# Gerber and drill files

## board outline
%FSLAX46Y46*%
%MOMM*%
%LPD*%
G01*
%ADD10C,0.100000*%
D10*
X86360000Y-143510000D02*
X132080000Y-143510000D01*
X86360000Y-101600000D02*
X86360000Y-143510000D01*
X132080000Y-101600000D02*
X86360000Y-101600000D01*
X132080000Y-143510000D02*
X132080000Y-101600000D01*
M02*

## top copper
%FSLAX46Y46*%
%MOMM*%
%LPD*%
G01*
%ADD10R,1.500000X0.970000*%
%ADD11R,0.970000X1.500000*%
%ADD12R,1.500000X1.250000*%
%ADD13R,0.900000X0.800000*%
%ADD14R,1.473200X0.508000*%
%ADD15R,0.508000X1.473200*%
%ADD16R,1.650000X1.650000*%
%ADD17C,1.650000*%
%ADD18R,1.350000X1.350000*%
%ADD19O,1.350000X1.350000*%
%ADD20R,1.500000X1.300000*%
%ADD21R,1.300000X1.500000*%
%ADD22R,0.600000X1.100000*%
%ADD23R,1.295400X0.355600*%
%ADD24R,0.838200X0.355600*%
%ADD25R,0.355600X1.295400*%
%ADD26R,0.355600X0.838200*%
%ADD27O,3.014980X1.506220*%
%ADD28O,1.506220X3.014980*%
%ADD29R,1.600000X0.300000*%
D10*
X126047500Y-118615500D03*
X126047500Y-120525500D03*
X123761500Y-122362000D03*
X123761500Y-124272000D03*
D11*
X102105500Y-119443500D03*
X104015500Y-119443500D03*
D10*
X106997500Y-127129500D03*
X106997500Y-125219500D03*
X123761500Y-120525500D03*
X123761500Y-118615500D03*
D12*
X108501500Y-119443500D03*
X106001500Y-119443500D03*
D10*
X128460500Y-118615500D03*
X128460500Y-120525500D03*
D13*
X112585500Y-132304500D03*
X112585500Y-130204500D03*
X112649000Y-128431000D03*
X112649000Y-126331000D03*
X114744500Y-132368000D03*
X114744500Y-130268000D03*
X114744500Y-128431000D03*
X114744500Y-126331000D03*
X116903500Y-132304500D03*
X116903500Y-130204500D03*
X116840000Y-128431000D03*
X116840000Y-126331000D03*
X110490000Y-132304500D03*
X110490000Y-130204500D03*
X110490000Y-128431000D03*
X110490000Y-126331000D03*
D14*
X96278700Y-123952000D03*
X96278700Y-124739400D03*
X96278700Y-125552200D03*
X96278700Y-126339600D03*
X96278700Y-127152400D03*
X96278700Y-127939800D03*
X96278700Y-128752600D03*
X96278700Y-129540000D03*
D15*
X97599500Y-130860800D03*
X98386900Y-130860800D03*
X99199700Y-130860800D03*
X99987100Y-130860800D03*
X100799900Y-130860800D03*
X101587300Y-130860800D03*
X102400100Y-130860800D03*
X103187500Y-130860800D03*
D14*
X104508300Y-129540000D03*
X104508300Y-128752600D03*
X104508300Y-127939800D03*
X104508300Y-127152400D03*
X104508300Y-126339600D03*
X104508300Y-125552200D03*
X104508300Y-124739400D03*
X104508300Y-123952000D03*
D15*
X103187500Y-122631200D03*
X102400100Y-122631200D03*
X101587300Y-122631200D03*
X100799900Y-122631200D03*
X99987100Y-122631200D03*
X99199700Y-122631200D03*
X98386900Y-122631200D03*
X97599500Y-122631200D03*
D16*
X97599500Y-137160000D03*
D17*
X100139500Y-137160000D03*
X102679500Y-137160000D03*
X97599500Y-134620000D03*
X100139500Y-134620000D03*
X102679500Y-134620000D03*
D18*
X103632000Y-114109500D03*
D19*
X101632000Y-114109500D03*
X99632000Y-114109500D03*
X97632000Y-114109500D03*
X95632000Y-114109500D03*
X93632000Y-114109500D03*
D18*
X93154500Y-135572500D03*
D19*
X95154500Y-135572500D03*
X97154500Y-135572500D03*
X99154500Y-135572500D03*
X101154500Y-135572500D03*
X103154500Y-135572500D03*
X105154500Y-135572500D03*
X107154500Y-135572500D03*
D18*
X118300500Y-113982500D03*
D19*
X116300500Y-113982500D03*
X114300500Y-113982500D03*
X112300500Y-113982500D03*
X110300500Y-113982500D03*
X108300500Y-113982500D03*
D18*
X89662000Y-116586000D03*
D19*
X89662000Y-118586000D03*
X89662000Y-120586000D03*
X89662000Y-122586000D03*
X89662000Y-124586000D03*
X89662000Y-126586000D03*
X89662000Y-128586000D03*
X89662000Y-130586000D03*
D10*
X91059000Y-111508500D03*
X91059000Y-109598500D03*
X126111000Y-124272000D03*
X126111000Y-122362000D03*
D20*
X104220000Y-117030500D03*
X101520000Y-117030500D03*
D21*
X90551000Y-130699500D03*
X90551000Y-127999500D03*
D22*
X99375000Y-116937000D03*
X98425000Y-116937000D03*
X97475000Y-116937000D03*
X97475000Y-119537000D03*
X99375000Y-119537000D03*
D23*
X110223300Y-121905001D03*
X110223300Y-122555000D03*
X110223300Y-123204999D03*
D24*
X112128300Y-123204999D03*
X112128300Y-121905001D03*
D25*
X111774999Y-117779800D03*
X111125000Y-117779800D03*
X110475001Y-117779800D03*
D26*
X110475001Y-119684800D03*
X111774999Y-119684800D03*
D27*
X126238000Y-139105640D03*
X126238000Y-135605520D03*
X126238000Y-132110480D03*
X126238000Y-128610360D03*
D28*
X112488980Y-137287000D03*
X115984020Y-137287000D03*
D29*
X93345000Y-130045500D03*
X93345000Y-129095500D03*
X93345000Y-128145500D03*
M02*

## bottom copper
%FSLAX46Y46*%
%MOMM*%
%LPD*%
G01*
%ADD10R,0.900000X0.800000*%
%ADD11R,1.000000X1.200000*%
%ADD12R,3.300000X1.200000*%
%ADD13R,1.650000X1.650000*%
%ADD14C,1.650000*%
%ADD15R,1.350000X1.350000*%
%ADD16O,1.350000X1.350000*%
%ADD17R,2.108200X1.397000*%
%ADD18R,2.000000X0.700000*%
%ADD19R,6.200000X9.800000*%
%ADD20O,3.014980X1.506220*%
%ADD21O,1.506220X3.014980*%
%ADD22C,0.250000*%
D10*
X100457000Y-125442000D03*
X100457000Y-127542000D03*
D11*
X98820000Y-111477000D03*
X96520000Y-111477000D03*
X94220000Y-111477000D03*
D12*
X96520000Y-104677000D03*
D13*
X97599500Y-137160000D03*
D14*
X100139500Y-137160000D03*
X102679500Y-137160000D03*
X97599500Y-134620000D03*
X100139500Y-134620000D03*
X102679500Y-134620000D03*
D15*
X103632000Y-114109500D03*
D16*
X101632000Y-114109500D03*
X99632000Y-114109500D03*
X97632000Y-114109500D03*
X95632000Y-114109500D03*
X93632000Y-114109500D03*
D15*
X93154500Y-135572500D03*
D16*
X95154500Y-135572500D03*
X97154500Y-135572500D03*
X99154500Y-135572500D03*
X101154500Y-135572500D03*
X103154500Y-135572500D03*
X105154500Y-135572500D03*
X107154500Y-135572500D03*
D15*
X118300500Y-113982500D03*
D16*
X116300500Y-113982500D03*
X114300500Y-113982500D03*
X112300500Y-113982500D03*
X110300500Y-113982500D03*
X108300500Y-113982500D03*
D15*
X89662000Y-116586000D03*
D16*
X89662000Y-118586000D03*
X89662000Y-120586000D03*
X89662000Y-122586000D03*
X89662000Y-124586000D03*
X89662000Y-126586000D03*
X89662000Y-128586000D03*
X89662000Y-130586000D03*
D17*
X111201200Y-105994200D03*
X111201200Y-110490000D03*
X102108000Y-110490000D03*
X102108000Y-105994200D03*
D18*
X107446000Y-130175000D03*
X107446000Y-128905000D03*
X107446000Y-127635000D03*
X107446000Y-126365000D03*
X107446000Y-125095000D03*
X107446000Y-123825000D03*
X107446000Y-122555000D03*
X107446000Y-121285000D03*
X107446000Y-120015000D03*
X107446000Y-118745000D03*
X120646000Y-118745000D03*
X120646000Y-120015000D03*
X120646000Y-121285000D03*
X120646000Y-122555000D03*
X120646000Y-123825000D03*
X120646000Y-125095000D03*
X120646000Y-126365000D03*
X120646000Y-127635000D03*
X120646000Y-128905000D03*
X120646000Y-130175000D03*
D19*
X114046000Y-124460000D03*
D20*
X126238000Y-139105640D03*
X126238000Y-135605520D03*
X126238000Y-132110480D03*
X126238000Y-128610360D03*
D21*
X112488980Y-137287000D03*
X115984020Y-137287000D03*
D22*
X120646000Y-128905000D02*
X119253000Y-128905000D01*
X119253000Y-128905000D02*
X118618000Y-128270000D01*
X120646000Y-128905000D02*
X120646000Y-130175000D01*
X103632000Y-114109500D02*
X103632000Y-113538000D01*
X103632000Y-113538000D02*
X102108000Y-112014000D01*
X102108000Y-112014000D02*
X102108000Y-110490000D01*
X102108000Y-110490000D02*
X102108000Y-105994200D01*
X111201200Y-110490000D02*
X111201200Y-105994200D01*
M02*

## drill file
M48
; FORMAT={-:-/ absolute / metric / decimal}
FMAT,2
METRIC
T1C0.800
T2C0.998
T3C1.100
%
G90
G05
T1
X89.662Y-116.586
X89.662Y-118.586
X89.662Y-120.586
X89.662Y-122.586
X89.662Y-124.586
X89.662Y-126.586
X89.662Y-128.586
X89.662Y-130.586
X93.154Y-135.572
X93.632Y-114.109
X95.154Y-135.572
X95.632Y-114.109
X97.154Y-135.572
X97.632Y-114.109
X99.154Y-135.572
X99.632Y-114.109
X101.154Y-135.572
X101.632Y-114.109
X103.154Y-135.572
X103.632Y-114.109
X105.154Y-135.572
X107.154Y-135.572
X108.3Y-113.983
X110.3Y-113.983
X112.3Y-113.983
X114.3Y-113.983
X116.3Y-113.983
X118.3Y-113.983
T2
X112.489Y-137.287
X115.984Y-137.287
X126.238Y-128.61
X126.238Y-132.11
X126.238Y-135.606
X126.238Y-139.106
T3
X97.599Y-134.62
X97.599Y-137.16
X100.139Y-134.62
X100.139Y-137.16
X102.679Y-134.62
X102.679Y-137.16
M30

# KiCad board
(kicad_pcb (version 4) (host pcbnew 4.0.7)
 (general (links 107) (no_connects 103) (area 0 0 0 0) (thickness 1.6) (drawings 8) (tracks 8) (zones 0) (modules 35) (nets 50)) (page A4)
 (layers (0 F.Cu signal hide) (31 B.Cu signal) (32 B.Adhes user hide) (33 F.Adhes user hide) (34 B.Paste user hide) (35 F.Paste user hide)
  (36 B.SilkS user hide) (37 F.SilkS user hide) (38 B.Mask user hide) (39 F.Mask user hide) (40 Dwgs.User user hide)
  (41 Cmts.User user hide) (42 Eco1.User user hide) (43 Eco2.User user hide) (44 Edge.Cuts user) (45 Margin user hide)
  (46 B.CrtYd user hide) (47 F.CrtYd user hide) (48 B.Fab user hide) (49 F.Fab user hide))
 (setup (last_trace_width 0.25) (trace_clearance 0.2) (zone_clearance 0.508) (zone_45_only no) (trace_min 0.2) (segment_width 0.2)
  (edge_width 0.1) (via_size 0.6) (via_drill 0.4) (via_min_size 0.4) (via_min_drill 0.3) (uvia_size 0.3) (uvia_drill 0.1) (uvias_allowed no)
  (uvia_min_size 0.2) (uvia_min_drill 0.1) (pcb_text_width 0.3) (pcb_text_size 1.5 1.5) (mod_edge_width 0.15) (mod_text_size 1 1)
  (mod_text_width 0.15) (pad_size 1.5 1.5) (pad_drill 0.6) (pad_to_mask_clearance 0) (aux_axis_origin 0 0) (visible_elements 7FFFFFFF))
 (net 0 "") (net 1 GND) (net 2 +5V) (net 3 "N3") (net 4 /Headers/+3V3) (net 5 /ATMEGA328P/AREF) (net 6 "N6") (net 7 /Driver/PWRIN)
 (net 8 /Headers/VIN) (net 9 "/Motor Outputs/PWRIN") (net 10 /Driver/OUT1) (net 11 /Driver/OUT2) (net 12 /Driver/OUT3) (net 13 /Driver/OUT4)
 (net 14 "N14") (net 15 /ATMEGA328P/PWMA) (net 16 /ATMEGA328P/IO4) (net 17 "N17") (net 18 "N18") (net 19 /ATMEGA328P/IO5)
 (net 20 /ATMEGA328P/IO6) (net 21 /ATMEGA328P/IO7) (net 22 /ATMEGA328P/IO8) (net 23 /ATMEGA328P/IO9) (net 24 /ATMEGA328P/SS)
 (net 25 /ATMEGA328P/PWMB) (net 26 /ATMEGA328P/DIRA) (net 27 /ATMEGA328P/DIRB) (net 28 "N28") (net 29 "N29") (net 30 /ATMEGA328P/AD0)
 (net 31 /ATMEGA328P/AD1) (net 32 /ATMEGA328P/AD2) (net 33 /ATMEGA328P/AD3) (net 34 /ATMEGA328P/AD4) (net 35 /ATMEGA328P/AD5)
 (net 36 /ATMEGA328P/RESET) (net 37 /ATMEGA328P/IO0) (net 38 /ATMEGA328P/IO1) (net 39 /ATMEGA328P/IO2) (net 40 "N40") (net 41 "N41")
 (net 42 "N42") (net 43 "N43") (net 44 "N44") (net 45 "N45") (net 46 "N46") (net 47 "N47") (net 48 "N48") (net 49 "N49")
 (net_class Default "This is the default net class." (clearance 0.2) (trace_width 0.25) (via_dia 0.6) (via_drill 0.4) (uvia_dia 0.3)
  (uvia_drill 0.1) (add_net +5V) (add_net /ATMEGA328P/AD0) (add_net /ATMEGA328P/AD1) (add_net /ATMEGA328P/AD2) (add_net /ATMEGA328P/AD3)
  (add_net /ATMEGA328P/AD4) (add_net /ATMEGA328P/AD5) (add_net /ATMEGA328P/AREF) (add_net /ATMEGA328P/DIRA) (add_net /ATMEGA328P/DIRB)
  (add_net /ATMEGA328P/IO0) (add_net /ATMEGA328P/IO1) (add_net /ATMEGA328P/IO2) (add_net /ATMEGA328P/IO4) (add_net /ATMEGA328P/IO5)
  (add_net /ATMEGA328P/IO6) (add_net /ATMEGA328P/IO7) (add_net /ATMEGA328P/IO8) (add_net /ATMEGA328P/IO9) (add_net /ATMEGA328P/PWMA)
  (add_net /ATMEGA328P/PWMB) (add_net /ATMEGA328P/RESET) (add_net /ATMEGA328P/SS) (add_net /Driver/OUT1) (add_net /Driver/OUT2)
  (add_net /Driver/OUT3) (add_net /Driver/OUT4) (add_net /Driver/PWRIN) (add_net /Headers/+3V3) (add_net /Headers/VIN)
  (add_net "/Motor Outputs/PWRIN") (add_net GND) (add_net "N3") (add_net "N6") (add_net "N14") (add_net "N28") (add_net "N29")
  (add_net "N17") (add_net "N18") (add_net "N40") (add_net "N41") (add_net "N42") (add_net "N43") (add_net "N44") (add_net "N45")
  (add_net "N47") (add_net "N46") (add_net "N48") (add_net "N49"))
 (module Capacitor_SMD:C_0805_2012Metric (layer F.Cu) (at 126.0475 119.5705 270)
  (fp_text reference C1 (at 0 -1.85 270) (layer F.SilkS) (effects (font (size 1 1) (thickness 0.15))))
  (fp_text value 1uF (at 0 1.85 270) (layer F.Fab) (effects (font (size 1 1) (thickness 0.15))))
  (pad 1 smd rect (at -0.955 0 270) (size 0.97 1.5) (layers F.Cu F.Paste F.Mask) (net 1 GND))
  (pad 2 smd rect (at 0.955 0 270) (size 0.97 1.5) (layers F.Cu F.Paste F.Mask) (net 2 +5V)))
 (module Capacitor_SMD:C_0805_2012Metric (layer F.Cu) (at 123.7615 123.317 270)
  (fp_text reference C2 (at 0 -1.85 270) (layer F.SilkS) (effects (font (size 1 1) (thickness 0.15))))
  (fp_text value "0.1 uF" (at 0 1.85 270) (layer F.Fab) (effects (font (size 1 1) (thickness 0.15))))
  (pad 1 smd rect (at -0.955 0 270) (size 0.97 1.5) (layers F.Cu F.Paste F.Mask) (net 2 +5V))
  (pad 2 smd rect (at 0.955 0 270) (size 0.97 1.5) (layers F.Cu F.Paste F.Mask) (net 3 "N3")))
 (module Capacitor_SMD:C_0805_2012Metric (layer F.Cu) (at 103.0605 119.4435)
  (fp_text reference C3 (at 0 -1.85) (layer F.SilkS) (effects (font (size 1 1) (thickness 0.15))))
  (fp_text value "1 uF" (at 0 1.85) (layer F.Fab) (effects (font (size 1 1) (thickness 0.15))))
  (pad 1 smd rect (at -0.955 0) (size 0.97 1.5) (layers F.Cu F.Paste F.Mask) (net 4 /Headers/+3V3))
  (pad 2 smd rect (at 0.955 0) (size 0.97 1.5) (layers F.Cu F.Paste F.Mask) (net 1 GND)))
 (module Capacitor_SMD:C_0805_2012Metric (layer F.Cu) (at 106.9975 126.1745 90)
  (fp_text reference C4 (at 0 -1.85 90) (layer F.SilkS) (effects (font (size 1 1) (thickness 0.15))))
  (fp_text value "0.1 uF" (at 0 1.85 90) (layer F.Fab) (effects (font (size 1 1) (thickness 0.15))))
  (pad 1 smd rect (at -0.955 0 90) (size 0.97 1.5) (layers F.Cu F.Paste F.Mask) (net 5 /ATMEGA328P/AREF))
  (pad 2 smd rect (at 0.955 0 90) (size 0.97 1.5) (layers F.Cu F.Paste F.Mask) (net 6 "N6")))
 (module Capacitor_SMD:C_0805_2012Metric (layer F.Cu) (at 123.7615 119.5705 90)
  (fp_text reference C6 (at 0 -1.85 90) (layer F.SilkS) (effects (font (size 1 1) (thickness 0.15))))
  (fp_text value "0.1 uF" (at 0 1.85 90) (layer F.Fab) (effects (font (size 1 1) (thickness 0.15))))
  (pad 1 smd rect (at -0.955 0 90) (size 0.97 1.5) (layers F.Cu F.Paste F.Mask) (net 2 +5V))
  (pad 2 smd rect (at 0.955 0 90) (size 0.97 1.5) (layers F.Cu F.Paste F.Mask) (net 1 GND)))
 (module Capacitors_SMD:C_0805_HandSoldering (layer F.Cu) (at 107.2515 119.4435 180)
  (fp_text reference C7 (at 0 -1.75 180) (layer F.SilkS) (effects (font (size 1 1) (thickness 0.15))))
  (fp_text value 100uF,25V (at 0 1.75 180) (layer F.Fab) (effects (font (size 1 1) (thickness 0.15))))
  (pad 1 smd rect (at -1.25 0 180) (size 1.5 1.25) (layers F.Cu F.Paste F.Mask) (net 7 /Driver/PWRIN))
  (pad 2 smd rect (at 1.25 0 180) (size 1.5 1.25) (layers F.Cu F.Paste F.Mask) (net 1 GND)))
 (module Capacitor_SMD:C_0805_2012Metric (layer F.Cu) (at 128.4605 119.5705 270)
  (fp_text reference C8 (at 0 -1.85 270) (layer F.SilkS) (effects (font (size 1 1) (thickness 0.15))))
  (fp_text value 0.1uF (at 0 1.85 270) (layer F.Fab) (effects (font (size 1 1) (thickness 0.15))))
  (pad 1 smd rect (at -0.955 0 270) (size 0.97 1.5) (layers F.Cu F.Paste F.Mask) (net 1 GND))
  (pad 2 smd rect (at 0.955 0 270) (size 0.97 1.5) (layers F.Cu F.Paste F.Mask) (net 2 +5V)))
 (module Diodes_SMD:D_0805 (layer B.Cu) (at 100.457 126.492 270)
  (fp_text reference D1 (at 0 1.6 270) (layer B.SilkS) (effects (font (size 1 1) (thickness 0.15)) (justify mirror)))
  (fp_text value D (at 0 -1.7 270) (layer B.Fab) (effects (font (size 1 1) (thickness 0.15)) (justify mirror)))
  (pad 1 smd rect (at -1.05 0 270) (size 0.8 0.9) (layers B.Cu B.Paste B.Mask) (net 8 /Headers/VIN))
  (pad 2 smd rect (at 1.05 0 270) (size 0.8 0.9) (layers B.Cu B.Paste B.Mask) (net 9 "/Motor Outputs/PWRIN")))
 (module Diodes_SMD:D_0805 (layer F.Cu) (at 112.5855 131.2545 90)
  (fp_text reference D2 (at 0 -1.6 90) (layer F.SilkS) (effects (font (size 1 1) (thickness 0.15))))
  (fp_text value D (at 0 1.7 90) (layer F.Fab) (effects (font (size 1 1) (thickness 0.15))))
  (pad 1 smd rect (at -1.05 0 90) (size 0.8 0.9) (layers F.Cu F.Paste F.Mask) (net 9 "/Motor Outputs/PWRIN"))
  (pad 2 smd rect (at 1.05 0 90) (size 0.8 0.9) (layers F.Cu F.Paste F.Mask) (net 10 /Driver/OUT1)))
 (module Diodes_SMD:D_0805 (layer F.Cu) (at 112.649 127.381 90)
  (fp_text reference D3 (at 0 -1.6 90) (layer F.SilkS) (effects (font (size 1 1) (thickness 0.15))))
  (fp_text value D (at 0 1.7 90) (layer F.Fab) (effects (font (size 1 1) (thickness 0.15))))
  (pad 1 smd rect (at -1.05 0 90) (size 0.8 0.9) (layers F.Cu F.Paste F.Mask) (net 10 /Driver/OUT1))
  (pad 2 smd rect (at 1.05 0 90) (size 0.8 0.9) (layers F.Cu F.Paste F.Mask) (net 1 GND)))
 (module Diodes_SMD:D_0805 (layer F.Cu) (at 114.7445 131.318 90)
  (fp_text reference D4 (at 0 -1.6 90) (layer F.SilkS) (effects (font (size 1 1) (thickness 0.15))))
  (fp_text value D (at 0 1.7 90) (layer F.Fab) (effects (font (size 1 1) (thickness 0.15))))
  (pad 1 smd rect (at -1.05 0 90) (size 0.8 0.9) (layers F.Cu F.Paste F.Mask) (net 9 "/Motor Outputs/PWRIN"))
  (pad 2 smd rect (at 1.05 0 90) (size 0.8 0.9) (layers F.Cu F.Paste F.Mask) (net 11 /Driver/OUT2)))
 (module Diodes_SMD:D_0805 (layer F.Cu) (at 114.7445 127.381 90)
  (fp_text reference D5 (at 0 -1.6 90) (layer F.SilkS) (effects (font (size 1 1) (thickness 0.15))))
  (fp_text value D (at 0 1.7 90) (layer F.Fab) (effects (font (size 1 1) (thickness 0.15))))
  (pad 1 smd rect (at -1.05 0 90) (size 0.8 0.9) (layers F.Cu F.Paste F.Mask) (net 11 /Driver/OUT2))
  (pad 2 smd rect (at 1.05 0 90) (size 0.8 0.9) (layers F.Cu F.Paste F.Mask) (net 1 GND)))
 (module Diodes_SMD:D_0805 (layer F.Cu) (at 116.9035 131.2545 90)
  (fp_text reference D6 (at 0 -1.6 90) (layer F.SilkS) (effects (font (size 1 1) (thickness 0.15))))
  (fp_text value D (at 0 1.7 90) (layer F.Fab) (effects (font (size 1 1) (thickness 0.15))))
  (pad 1 smd rect (at -1.05 0 90) (size 0.8 0.9) (layers F.Cu F.Paste F.Mask) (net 9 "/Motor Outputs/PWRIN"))
  (pad 2 smd rect (at 1.05 0 90) (size 0.8 0.9) (layers F.Cu F.Paste F.Mask) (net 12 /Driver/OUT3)))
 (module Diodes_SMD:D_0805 (layer F.Cu) (at 116.84 127.381 90)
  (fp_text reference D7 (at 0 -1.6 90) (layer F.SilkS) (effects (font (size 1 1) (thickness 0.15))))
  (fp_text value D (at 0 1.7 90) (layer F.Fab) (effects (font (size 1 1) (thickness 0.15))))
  (pad 1 smd rect (at -1.05 0 90) (size 0.8 0.9) (layers F.Cu F.Paste F.Mask) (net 12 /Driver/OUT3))
  (pad 2 smd rect (at 1.05 0 90) (size 0.8 0.9) (layers F.Cu F.Paste F.Mask) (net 1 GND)))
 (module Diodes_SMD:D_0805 (layer F.Cu) (at 110.49 131.2545 90)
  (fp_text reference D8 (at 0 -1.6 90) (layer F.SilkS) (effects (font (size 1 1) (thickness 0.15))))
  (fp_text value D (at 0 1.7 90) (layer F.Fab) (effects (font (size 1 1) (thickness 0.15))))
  (pad 1 smd rect (at -1.05 0 90) (size 0.8 0.9) (layers F.Cu F.Paste F.Mask) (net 9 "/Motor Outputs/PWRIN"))
  (pad 2 smd rect (at 1.05 0 90) (size 0.8 0.9) (layers F.Cu F.Paste F.Mask) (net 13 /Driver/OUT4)))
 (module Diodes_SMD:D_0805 (layer F.Cu) (at 110.49 127.381 90)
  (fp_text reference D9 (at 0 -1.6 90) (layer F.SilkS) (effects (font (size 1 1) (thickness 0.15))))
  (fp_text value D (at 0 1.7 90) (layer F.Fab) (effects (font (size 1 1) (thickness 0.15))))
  (pad 1 smd rect (at -1.05 0 90) (size 0.8 0.9) (layers F.Cu F.Paste F.Mask) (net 13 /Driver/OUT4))
  (pad 2 smd rect (at 1.05 0 90) (size 0.8 0.9) (layers F.Cu F.Paste F.Mask) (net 1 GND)))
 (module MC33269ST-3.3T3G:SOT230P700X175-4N (layer B.Cu) (at 96.52 108.077 90)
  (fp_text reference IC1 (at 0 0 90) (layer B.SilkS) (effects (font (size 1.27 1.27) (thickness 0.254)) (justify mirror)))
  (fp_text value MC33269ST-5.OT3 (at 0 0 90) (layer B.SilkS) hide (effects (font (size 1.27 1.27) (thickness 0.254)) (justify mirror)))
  (pad 1 smd rect (at -3.4 2.3) (size 1 1.2) (layers B.Cu B.Paste B.Mask) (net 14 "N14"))
  (pad 2 smd rect (at -3.4 0) (size 1 1.2) (layers B.Cu B.Paste B.Mask) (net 2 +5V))
  (pad 3 smd rect (at -3.4 -2.3) (size 1 1.2) (layers B.Cu B.Paste B.Mask) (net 8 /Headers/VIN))
  (pad 4 smd rect (at 3.4 0 90) (size 1.2 3.3) (layers B.Cu B.Paste B.Mask) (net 2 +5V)))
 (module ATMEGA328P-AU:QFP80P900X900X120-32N (layer F.Cu) (at 100.3935 126.746)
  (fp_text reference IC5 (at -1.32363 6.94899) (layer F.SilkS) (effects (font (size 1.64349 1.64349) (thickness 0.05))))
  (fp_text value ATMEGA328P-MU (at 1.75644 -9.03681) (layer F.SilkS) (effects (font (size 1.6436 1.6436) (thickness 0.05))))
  (pad 1 smd rect (at -4.1148 -2.794 270) (size 0.508 1.4732) (layers F.Cu F.Paste F.Mask) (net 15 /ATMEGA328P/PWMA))
  (pad 2 smd rect (at -4.1148 -2.0066 270) (size 0.508 1.4732) (layers F.Cu F.Paste F.Mask) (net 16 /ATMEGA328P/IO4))
  (pad 3 smd rect (at -4.1148 -1.1938 270) (size 0.508 1.4732) (layers F.Cu F.Paste F.Mask) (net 1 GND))
  (pad 4 smd rect (at -4.1148 -0.4064 270) (size 0.508 1.4732) (layers F.Cu F.Paste F.Mask) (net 2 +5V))
  (pad 5 smd rect (at -4.1148 0.4064 270) (size 0.508 1.4732) (layers F.Cu F.Paste F.Mask) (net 1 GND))
  (pad 6 smd rect (at -4.1148 1.1938 270) (size 0.508 1.4732) (layers F.Cu F.Paste F.Mask) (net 2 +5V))
  (pad 7 smd rect (at -4.1148 2.0066 270) (size 0.508 1.4732) (layers F.Cu F.Paste F.Mask) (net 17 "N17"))
  (pad 8 smd rect (at -4.1148 2.794 270) (size 0.508 1.4732) (layers F.Cu F.Paste F.Mask) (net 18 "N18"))
  (pad 9 smd rect (at -2.794 4.1148 180) (size 0.508 1.4732) (layers F.Cu F.Paste F.Mask) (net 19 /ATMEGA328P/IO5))
  (pad 10 smd rect (at -2.0066 4.1148 180) (size 0.508 1.4732) (layers F.Cu F.Paste F.Mask) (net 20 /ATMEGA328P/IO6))
  (pad 11 smd rect (at -1.1938 4.1148 180) (size 0.508 1.4732) (layers F.Cu F.Paste F.Mask) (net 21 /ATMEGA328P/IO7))
  (pad 12 smd rect (at -0.4064 4.1148 180) (size 0.508 1.4732) (layers F.Cu F.Paste F.Mask) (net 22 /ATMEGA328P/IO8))
  (pad 13 smd rect (at 0.4064 4.1148 180) (size 0.508 1.4732) (layers F.Cu F.Paste F.Mask) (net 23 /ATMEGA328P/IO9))
  (pad 14 smd rect (at 1.1938 4.1148 180) (size 0.508 1.4732) (layers F.Cu F.Paste F.Mask) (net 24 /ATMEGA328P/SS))
  (pad 15 smd rect (at 2.0066 4.1148 180) (size 0.508 1.4732) (layers F.Cu F.Paste F.Mask) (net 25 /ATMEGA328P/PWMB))
  (pad 16 smd rect (at 2.794 4.1148 180) (size 0.508 1.4732) (layers F.Cu F.Paste F.Mask) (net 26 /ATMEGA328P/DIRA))
  (pad 17 smd rect (at 4.1148 2.794 270) (size 0.508 1.4732) (layers F.Cu F.Paste F.Mask) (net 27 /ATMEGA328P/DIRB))
  (pad 18 smd rect (at 4.1148 2.0066 270) (size 0.508 1.4732) (layers F.Cu F.Paste F.Mask) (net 2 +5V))
  (pad 19 smd rect (at 4.1148 1.1938 270) (size 0.508 1.4732) (layers F.Cu F.Paste F.Mask) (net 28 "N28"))
  (pad 20 smd rect (at 4.1148 0.4064 270) (size 0.508 1.4732) (layers F.Cu F.Paste F.Mask) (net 5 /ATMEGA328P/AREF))
  (pad 21 smd rect (at 4.1148 -0.4064 270) (size 0.508 1.4732) (layers F.Cu F.Paste F.Mask) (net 1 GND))
  (pad 22 smd rect (at 4.1148 -1.1938 270) (size 0.508 1.4732) (layers F.Cu F.Paste F.Mask) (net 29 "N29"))
  (pad 23 smd rect (at 4.1148 -2.0066 270) (size 0.508 1.4732) (layers F.Cu F.Paste F.Mask) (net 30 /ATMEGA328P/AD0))
  (pad 24 smd rect (at 4.1148 -2.794 270) (size 0.508 1.4732) (layers F.Cu F.Paste F.Mask) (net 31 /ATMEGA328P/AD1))
  (pad 25 smd rect (at 2.794 -4.1148 180) (size 0.508 1.4732) (layers F.Cu F.Paste F.Mask) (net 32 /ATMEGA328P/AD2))
  (pad 26 smd rect (at 2.0066 -4.1148 180) (size 0.508 1.4732) (layers F.Cu F.Paste F.Mask) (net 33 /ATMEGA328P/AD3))
  (pad 27 smd rect (at 1.1938 -4.1148 180) (size 0.508 1.4732) (layers F.Cu F.Paste F.Mask) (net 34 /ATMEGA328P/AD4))
  (pad 28 smd rect (at 0.4064 -4.1148 180) (size 0.508 1.4732) (layers F.Cu F.Paste F.Mask) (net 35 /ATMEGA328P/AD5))
  (pad 29 smd rect (at -0.4064 -4.1148 180) (size 0.508 1.4732) (layers F.Cu F.Paste F.Mask) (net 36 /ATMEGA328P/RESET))
  (pad 30 smd rect (at -1.1938 -4.1148 180) (size 0.508 1.4732) (layers F.Cu F.Paste F.Mask) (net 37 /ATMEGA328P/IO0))
  (pad 31 smd rect (at -2.0066 -4.1148 180) (size 0.508 1.4732) (layers F.Cu F.Paste F.Mask) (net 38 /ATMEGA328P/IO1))
  (pad 32 smd rect (at -2.794 -4.1148 180) (size 0.508 1.4732) (layers F.Cu F.Paste F.Mask) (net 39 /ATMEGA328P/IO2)))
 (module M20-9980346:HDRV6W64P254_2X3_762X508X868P (layer F.Cu) (at 97.5995 137.16)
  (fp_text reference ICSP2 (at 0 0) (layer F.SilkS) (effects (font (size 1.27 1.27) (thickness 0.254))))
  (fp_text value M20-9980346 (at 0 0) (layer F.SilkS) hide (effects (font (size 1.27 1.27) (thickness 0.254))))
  (pad 1 thru_hole rect (at 0 0 90) (size 1.65 1.65) (drill 1.1) (layers *.Cu *.Mask F.SilkS) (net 26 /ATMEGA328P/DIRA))
  (pad 3 thru_hole circle (at 2.54 0 90) (size 1.65 1.65) (drill 1.1) (layers *.Cu *.Mask F.SilkS) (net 27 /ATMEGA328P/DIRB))
  (pad 5 thru_hole circle (at 5.08 0 90) (size 1.65 1.65) (drill 1.1) (layers *.Cu *.Mask F.SilkS) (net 36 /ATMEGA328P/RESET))
  (pad 2 thru_hole circle (at 0 -2.54 90) (size 1.65 1.65) (drill 1.1) (layers *.Cu *.Mask F.SilkS) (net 2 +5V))
  (pad 4 thru_hole circle (at 2.54 -2.54 90) (size 1.65 1.65) (drill 1.1) (layers *.Cu *.Mask F.SilkS) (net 25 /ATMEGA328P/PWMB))
  (pad 6 thru_hole circle (at 5.08 -2.54 90) (size 1.65 1.65) (drill 1.1) (layers *.Cu *.Mask F.SilkS) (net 1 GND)))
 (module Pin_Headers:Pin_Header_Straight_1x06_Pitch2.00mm (layer B.Cu) (at 103.632 114.1095 90)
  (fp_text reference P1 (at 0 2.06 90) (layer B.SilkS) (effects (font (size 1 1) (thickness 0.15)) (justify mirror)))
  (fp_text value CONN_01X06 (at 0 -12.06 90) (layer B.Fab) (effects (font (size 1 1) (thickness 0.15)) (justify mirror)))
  (pad 1 thru_hole rect (at 0 0 90) (size 1.35 1.35) (drill 0.8) (layers *.Cu *.Mask) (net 36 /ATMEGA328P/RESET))
  (pad 2 thru_hole oval (at 0 -2 90) (size 1.35 1.35) (drill 0.8) (layers *.Cu *.Mask) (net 4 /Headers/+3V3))
  (pad 3 thru_hole oval (at 0 -4 90) (size 1.35 1.35) (drill 0.8) (layers *.Cu *.Mask) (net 2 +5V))
  (pad 4 thru_hole oval (at 0 -6 90) (size 1.35 1.35) (drill 0.8) (layers *.Cu *.Mask) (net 1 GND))
  (pad 5 thru_hole oval (at 0 -8 90) (size 1.35 1.35) (drill 0.8) (layers *.Cu *.Mask) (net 1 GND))
  (pad 6 thru_hole oval (at 0 -10 90) (size 1.35 1.35) (drill 0.8) (layers *.Cu *.Mask) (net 8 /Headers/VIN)))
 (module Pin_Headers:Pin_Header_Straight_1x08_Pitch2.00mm (layer B.Cu) (at 93.1545 135.5725 270)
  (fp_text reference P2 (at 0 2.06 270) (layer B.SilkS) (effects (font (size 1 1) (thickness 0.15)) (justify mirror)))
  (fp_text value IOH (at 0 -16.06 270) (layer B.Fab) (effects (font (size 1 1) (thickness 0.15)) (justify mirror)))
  (pad 1 thru_hole rect (at 0 0 270) (size 1.35 1.35) (drill 0.8) (layers *.Cu *.Mask) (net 22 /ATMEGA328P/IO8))
  (pad 2 thru_hole oval (at 0 -2 270) (size 1.35 1.35) (drill 0.8) (layers *.Cu *.Mask) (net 23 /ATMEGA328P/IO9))
  (pad 3 thru_hole oval (at 0 -4 270) (size 1.35 1.35) (drill 0.8) (layers *.Cu *.Mask) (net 24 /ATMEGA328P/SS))
  (pad 4 thru_hole oval (at 0 -6 270) (size 1.35 1.35) (drill 0.8) (layers *.Cu *.Mask) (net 25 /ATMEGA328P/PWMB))
  (pad 5 thru_hole oval (at 0 -8 270) (size 1.35 1.35) (drill 0.8) (layers *.Cu *.Mask) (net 26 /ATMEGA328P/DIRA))
  (pad 6 thru_hole oval (at 0 -10 270) (size 1.35 1.35) (drill 0.8) (layers *.Cu *.Mask) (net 27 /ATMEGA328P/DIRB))
  (pad 7 thru_hole oval (at 0 -12 270) (size 1.35 1.35) (drill 0.8) (layers *.Cu *.Mask) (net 1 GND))
  (pad 8 thru_hole oval (at 0 -14 270) (size 1.35 1.35) (drill 0.8) (layers *.Cu *.Mask) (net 5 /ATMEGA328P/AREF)))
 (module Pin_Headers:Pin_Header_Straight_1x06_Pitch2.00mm (layer F.Cu) (at 118.3005 113.9825 270)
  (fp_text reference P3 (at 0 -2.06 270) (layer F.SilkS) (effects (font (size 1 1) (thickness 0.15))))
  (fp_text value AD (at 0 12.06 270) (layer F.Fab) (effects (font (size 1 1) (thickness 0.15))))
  (pad 1 thru_hole rect (at 0 0 270) (size 1.35 1.35) (drill 0.8) (layers *.Cu *.Mask) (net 30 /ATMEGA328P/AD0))
  (pad 2 thru_hole oval (at 0 2 270) (size 1.35 1.35) (drill 0.8) (layers *.Cu *.Mask) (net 31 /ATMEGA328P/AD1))
  (pad 3 thru_hole oval (at 0 4 270) (size 1.35 1.35) (drill 0.8) (layers *.Cu *.Mask) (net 32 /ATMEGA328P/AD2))
  (pad 4 thru_hole oval (at 0 6 270) (size 1.35 1.35) (drill 0.8) (layers *.Cu *.Mask) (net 33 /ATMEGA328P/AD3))
  (pad 5 thru_hole oval (at 0 8 270) (size 1.35 1.35) (drill 0.8) (layers *.Cu *.Mask) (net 34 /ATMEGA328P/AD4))
  (pad 6 thru_hole oval (at 0 10 270) (size 1.35 1.35) (drill 0.8) (layers *.Cu *.Mask) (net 35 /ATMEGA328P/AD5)))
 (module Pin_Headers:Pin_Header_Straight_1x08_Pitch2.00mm (layer B.Cu) (at 89.662 116.586 180)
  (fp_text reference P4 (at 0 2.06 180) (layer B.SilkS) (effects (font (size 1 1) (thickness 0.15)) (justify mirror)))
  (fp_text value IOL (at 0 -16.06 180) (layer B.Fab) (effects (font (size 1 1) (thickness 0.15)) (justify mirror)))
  (pad 1 thru_hole rect (at 0 0 180) (size 1.35 1.35) (drill 0.8) (layers *.Cu *.Mask) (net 37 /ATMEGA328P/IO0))
  (pad 2 thru_hole oval (at 0 -2 180) (size 1.35 1.35) (drill 0.8) (layers *.Cu *.Mask) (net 38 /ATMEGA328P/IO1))
  (pad 3 thru_hole oval (at 0 -4 180) (size 1.35 1.35) (drill 0.8) (layers *.Cu *.Mask) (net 39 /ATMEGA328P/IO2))
  (pad 4 thru_hole oval (at 0 -6 180) (size 1.35 1.35) (drill 0.8) (layers *.Cu *.Mask) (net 15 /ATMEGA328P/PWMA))
  (pad 5 thru_hole oval (at 0 -8 180) (size 1.35 1.35) (drill 0.8) (layers *.Cu *.Mask) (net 16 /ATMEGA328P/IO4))
  (pad 6 thru_hole oval (at 0 -10 180) (size 1.35 1.35) (drill 0.8) (layers *.Cu *.Mask) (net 19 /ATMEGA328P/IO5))
  (pad 7 thru_hole oval (at 0 -12 180) (size 1.35 1.35) (drill 0.8) (layers *.Cu *.Mask) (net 20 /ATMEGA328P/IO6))
  (pad 8 thru_hole oval (at 0 -14 180) (size 1.35 1.35) (drill 0.8) (layers *.Cu *.Mask) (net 21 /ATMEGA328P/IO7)))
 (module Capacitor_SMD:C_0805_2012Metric (layer F.Cu) (at 91.059 110.5535 90)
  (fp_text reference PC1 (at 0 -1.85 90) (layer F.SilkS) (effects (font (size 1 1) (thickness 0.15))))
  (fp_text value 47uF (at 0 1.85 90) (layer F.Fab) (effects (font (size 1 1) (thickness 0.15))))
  (pad 1 smd rect (at -0.955 0 90) (size 0.97 1.5) (layers F.Cu F.Paste F.Mask) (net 8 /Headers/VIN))
  (pad 2 smd rect (at 0.955 0 90) (size 0.97 1.5) (layers F.Cu F.Paste F.Mask) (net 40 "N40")))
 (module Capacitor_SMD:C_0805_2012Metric (layer F.Cu) (at 126.111 123.317 90)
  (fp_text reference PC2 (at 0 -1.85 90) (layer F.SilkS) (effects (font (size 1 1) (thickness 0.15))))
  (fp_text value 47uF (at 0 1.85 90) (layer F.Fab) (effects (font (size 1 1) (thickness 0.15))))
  (pad 1 smd rect (at -0.955 0 90) (size 0.97 1.5) (layers F.Cu F.Paste F.Mask) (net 2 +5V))
  (pad 2 smd rect (at 0.955 0 90) (size 0.97 1.5) (layers F.Cu F.Paste F.Mask) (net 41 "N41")))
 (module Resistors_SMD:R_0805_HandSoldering (layer F.Cu) (at 102.87 117.0305 180)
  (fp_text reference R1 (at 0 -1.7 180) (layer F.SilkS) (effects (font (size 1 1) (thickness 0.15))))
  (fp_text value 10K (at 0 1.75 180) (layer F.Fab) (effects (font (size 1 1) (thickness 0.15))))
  (pad 1 smd rect (at -1.35 0 180) (size 1.5 1.3) (layers F.Cu F.Paste F.Mask) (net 36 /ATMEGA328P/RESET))
  (pad 2 smd rect (at 1.35 0 180) (size 1.5 1.3) (layers F.Cu F.Paste F.Mask) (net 2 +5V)))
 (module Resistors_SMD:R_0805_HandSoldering (layer F.Cu) (at 90.551 129.3495 90)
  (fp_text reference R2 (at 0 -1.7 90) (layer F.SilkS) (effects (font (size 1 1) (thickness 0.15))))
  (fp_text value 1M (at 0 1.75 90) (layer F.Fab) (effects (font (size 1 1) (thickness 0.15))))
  (pad 1 smd rect (at -1.35 0 90) (size 1.5 1.3) (layers F.Cu F.Paste F.Mask) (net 18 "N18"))
  (pad 2 smd rect (at 1.35 0 90) (size 1.5 1.3) (layers F.Cu F.Paste F.Mask) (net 17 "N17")))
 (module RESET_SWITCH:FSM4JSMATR (layer B.Cu) (at 102.108 110.49 180)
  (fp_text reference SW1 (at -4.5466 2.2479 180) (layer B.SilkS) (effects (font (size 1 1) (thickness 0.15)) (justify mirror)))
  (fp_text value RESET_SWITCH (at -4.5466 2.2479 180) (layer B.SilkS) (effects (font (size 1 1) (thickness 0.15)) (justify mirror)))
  (pad 1 smd rect (at -9.0932 4.4958 180) (size 2.1082 1.397) (layers B.Cu B.Paste B.Mask) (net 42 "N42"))
  (pad 2 smd rect (at -9.0932 0 180) (size 2.1082 1.397) (layers B.Cu B.Paste B.Mask) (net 42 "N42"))
  (pad 3 smd rect (at 0 0 180) (size 2.1082 1.397) (layers B.Cu B.Paste B.Mask) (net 36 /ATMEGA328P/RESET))
  (pad 4 smd rect (at 0 4.4958 180) (size 2.1082 1.397) (layers B.Cu B.Paste B.Mask) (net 36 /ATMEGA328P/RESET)))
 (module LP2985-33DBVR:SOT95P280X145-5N (layer F.Cu) (at 98.425 118.237 270)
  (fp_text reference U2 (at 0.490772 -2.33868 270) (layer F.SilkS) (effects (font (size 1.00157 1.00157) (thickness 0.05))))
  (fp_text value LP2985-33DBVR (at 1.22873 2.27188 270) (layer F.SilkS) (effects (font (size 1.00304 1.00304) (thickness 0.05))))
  (pad 1 smd rect (at -1.3 -0.95 270) (size 1.1 0.6) (layers F.Cu F.Paste F.Mask) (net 2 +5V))
  (pad 2 smd rect (at -1.3 0 270) (size 1.1 0.6) (layers F.Cu F.Paste F.Mask) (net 1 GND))
  (pad 3 smd rect (at -1.3 0.95 270) (size 1.1 0.6) (layers F.Cu F.Paste F.Mask) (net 2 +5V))
  (pad 4 smd rect (at 1.3 0.95 90) (size 1.1 0.6) (layers F.Cu F.Paste F.Mask) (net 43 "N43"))
  (pad 5 smd rect (at 1.3 -0.95 90) (size 1.1 0.6) (layers F.Cu F.Paste F.Mask) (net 4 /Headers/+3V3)))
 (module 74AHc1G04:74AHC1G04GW (layer F.Cu) (at 111.0615 122.555)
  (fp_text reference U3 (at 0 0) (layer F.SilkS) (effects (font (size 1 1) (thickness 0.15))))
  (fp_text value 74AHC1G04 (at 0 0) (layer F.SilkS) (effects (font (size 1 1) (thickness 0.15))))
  (pad 1 smd rect (at -0.8382 -0.649999) (size 1.2954 0.3556) (layers F.Cu F.Paste F.Mask))
  (pad 2 smd rect (at -0.8382 0) (size 1.2954 0.3556) (layers F.Cu F.Paste F.Mask) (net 26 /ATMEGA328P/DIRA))
  (pad 3 smd rect (at -0.8382 0.649999) (size 1.2954 0.3556) (layers F.Cu F.Paste F.Mask) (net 1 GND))
  (pad 4 smd rect (at 1.0668 0.649999) (size 0.8382 0.3556) (layers F.Cu F.Paste F.Mask) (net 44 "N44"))
  (pad 5 smd rect (at 1.0668 -0.649999) (size 0.8382 0.3556) (layers F.Cu F.Paste F.Mask) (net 2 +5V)))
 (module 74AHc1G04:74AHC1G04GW (layer F.Cu) (at 111.125 118.618 270)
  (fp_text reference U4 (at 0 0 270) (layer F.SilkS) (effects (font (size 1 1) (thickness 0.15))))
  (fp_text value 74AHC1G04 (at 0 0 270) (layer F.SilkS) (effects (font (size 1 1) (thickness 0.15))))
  (pad 1 smd rect (at -0.8382 -0.649999 270) (size 1.2954 0.3556) (layers F.Cu F.Paste F.Mask))
  (pad 2 smd rect (at -0.8382 0 270) (size 1.2954 0.3556) (layers F.Cu F.Paste F.Mask) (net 27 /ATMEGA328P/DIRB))
  (pad 3 smd rect (at -0.8382 0.649999 270) (size 1.2954 0.3556) (layers F.Cu F.Paste F.Mask) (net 1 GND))
  (pad 4 smd rect (at 1.0668 0.649999 270) (size 0.8382 0.3556) (layers F.Cu F.Paste F.Mask) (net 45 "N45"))
  (pad 5 smd rect (at 1.0668 -0.649999 270) (size 0.8382 0.3556) (layers F.Cu F.Paste F.Mask) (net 2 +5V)))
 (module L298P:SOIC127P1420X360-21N (layer B.Cu) (at 114.046 124.46)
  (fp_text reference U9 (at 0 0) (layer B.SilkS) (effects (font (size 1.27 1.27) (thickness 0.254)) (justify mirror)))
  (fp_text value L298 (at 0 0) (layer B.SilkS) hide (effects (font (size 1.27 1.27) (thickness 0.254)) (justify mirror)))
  (pad 1 smd rect (at -6.6 5.715 270) (size 0.7 2) (layers B.Cu B.Paste B.Mask) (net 1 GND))
  (pad 2 smd rect (at -6.6 4.445 270) (size 0.7 2) (layers B.Cu B.Paste B.Mask) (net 1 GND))
  (pad 3 smd rect (at -6.6 3.175 270) (size 0.7 2) (layers B.Cu B.Paste B.Mask) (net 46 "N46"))
  (pad 4 smd rect (at -6.6 1.905 270) (size 0.7 2) (layers B.Cu B.Paste B.Mask) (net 10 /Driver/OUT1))
  (pad 5 smd rect (at -6.6 0.635 270) (size 0.7 2) (layers B.Cu B.Paste B.Mask) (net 11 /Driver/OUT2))
  (pad 6 smd rect (at -6.6 -0.635 270) (size 0.7 2) (layers B.Cu B.Paste B.Mask) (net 7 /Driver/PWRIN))
  (pad 7 smd rect (at -6.6 -1.905 270) (size 0.7 2) (layers B.Cu B.Paste B.Mask) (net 26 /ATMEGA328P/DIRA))
  (pad 8 smd rect (at -6.6 -3.175 270) (size 0.7 2) (layers B.Cu B.Paste B.Mask) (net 15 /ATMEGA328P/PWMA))
  (pad 9 smd rect (at -6.6 -4.445 270) (size 0.7 2) (layers B.Cu B.Paste B.Mask) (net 44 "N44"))
  (pad 10 smd rect (at -6.6 -5.715 270) (size 0.7 2) (layers B.Cu B.Paste B.Mask) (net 1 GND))
  (pad 11 smd rect (at 6.6 -5.715 270) (size 0.7 2) (layers B.Cu B.Paste B.Mask) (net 1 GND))
  (pad 12 smd rect (at 6.6 -4.445 270) (size 0.7 2) (layers B.Cu B.Paste B.Mask) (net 2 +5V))
  (pad 13 smd rect (at 6.6 -3.175 270) (size 0.7 2) (layers B.Cu B.Paste B.Mask) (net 27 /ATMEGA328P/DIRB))
  (pad 14 smd rect (at 6.6 -1.905 270) (size 0.7 2) (layers B.Cu B.Paste B.Mask) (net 25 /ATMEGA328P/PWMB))
  (pad 15 smd rect (at 6.6 -0.635 270) (size 0.7 2) (layers B.Cu B.Paste B.Mask) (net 45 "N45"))
  (pad 16 smd rect (at 6.6 0.635 270) (size 0.7 2) (layers B.Cu B.Paste B.Mask) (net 12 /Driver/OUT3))
  (pad 17 smd rect (at 6.6 1.905 270) (size 0.7 2) (layers B.Cu B.Paste B.Mask) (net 13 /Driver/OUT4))
  (pad 18 smd rect (at 6.6 3.175 270) (size 0.7 2) (layers B.Cu B.Paste B.Mask) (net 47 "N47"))
  (pad 19 smd rect (at 6.6 4.445 270) (size 0.7 2) (layers B.Cu B.Paste B.Mask) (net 1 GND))
  (pad 20 smd rect (at 6.6 5.715 270) (size 0.7 2) (layers B.Cu B.Paste B.Mask) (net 1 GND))
  (pad 21 smd rect (at 0 0) (size 6.2 9.8) (layers B.Cu B.Paste B.Mask)))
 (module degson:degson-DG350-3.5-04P (layer B.Cu) (at 126.238 133.858 90)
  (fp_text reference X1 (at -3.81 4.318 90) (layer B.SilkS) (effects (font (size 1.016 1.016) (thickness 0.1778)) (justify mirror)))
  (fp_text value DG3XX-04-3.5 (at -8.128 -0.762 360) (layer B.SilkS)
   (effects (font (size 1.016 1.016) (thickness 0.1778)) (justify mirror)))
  (pad 1 thru_hole oval (at -5.24764 0 270) (size 1.50622 3.01498) (drill 0.99822) (layers *.Cu *.Paste *.Mask) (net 10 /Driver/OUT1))
  (pad 2 thru_hole oval (at -1.74752 0 270) (size 1.50622 3.01498) (drill 0.99822) (layers *.Cu *.Paste *.Mask) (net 11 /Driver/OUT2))
  (pad 3 thru_hole oval (at 1.74752 0 270) (size 1.50622 3.01498) (drill 0.99822) (layers *.Cu *.Paste *.Mask) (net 12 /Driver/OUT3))
  (pad 4 thru_hole oval (at 5.24764 0 270) (size 1.50622 3.01498) (drill 0.99822) (layers *.Cu *.Paste *.Mask) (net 13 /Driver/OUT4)))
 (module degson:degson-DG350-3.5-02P (layer B.Cu) (at 114.2365 137.287)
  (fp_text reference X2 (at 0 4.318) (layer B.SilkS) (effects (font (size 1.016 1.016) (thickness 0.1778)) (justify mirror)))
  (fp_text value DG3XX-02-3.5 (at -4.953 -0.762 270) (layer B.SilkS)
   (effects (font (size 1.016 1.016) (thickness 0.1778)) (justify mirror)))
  (pad 1 thru_hole oval (at -1.74752 0 180) (size 1.50622 3.01498) (drill 0.99822) (layers *.Cu *.Paste *.Mask)
   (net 9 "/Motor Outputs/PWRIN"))
  (pad 2 thru_hole oval (at 1.74752 0 180) (size 1.50622 3.01498) (drill 0.99822) (layers *.Cu *.Paste *.Mask) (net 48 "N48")))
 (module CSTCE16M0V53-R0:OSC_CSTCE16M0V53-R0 (layer F.Cu) (at 93.345 129.0955 90)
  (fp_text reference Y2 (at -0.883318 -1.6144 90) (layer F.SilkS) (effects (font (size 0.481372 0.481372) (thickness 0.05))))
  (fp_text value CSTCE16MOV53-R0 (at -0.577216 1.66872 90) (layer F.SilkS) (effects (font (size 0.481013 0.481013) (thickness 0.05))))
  (pad 1 smd rect (at -0.95 0 180) (size 1.6 0.3) (layers F.Cu F.Paste F.Mask) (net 18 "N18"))
  (pad 2 smd rect (at 0 0 180) (size 1.6 0.3) (layers F.Cu F.Paste F.Mask) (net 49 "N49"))
  (pad 3 smd rect (at 0.95 0 180) (size 1.6 0.3) (layers F.Cu F.Paste F.Mask) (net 17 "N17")))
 (gr_line (start 86.36 143.51) (end 132.08 143.51) (angle 90) (layer Edge.Cuts) (width 0.1))
 (gr_line (start 86.36 101.6) (end 86.36 143.51) (angle 90) (layer Edge.Cuts) (width 0.1))
 (gr_line (start 132.08 101.6) (end 86.36 101.6) (angle 90) (layer Edge.Cuts) (width 0.1))
 (gr_line (start 132.08 143.51) (end 132.08 101.6) (angle 90) (layer Edge.Cuts) (width 0.1))
 (segment (start 120.646 128.905) (end 119.253 128.905) (width 0.25) (layer B.Cu) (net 1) (status 400000))
 (segment (start 119.253 128.905) (end 118.618 128.27) (width 0.25) (layer B.Cu) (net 1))
 (segment (start 120.646 128.905) (end 120.646 130.175) (width 0.25) (layer B.Cu) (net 1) (status C00000))
 (segment (start 103.632 114.1095) (end 103.632 113.538) (width 0.25) (layer B.Cu) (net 36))
 (segment (start 103.632 113.538) (end 102.108 112.014) (width 0.25) (layer B.Cu) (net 36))
 (segment (start 102.108 112.014) (end 102.108 110.49) (width 0.25) (layer B.Cu) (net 36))
 (segment (start 102.108 110.49) (end 102.108 105.9942) (width 0.25) (layer B.Cu) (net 36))
 (segment (start 111.2012 110.49) (end 111.2012 105.9942) (width 0.25) (layer B.Cu) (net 42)))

